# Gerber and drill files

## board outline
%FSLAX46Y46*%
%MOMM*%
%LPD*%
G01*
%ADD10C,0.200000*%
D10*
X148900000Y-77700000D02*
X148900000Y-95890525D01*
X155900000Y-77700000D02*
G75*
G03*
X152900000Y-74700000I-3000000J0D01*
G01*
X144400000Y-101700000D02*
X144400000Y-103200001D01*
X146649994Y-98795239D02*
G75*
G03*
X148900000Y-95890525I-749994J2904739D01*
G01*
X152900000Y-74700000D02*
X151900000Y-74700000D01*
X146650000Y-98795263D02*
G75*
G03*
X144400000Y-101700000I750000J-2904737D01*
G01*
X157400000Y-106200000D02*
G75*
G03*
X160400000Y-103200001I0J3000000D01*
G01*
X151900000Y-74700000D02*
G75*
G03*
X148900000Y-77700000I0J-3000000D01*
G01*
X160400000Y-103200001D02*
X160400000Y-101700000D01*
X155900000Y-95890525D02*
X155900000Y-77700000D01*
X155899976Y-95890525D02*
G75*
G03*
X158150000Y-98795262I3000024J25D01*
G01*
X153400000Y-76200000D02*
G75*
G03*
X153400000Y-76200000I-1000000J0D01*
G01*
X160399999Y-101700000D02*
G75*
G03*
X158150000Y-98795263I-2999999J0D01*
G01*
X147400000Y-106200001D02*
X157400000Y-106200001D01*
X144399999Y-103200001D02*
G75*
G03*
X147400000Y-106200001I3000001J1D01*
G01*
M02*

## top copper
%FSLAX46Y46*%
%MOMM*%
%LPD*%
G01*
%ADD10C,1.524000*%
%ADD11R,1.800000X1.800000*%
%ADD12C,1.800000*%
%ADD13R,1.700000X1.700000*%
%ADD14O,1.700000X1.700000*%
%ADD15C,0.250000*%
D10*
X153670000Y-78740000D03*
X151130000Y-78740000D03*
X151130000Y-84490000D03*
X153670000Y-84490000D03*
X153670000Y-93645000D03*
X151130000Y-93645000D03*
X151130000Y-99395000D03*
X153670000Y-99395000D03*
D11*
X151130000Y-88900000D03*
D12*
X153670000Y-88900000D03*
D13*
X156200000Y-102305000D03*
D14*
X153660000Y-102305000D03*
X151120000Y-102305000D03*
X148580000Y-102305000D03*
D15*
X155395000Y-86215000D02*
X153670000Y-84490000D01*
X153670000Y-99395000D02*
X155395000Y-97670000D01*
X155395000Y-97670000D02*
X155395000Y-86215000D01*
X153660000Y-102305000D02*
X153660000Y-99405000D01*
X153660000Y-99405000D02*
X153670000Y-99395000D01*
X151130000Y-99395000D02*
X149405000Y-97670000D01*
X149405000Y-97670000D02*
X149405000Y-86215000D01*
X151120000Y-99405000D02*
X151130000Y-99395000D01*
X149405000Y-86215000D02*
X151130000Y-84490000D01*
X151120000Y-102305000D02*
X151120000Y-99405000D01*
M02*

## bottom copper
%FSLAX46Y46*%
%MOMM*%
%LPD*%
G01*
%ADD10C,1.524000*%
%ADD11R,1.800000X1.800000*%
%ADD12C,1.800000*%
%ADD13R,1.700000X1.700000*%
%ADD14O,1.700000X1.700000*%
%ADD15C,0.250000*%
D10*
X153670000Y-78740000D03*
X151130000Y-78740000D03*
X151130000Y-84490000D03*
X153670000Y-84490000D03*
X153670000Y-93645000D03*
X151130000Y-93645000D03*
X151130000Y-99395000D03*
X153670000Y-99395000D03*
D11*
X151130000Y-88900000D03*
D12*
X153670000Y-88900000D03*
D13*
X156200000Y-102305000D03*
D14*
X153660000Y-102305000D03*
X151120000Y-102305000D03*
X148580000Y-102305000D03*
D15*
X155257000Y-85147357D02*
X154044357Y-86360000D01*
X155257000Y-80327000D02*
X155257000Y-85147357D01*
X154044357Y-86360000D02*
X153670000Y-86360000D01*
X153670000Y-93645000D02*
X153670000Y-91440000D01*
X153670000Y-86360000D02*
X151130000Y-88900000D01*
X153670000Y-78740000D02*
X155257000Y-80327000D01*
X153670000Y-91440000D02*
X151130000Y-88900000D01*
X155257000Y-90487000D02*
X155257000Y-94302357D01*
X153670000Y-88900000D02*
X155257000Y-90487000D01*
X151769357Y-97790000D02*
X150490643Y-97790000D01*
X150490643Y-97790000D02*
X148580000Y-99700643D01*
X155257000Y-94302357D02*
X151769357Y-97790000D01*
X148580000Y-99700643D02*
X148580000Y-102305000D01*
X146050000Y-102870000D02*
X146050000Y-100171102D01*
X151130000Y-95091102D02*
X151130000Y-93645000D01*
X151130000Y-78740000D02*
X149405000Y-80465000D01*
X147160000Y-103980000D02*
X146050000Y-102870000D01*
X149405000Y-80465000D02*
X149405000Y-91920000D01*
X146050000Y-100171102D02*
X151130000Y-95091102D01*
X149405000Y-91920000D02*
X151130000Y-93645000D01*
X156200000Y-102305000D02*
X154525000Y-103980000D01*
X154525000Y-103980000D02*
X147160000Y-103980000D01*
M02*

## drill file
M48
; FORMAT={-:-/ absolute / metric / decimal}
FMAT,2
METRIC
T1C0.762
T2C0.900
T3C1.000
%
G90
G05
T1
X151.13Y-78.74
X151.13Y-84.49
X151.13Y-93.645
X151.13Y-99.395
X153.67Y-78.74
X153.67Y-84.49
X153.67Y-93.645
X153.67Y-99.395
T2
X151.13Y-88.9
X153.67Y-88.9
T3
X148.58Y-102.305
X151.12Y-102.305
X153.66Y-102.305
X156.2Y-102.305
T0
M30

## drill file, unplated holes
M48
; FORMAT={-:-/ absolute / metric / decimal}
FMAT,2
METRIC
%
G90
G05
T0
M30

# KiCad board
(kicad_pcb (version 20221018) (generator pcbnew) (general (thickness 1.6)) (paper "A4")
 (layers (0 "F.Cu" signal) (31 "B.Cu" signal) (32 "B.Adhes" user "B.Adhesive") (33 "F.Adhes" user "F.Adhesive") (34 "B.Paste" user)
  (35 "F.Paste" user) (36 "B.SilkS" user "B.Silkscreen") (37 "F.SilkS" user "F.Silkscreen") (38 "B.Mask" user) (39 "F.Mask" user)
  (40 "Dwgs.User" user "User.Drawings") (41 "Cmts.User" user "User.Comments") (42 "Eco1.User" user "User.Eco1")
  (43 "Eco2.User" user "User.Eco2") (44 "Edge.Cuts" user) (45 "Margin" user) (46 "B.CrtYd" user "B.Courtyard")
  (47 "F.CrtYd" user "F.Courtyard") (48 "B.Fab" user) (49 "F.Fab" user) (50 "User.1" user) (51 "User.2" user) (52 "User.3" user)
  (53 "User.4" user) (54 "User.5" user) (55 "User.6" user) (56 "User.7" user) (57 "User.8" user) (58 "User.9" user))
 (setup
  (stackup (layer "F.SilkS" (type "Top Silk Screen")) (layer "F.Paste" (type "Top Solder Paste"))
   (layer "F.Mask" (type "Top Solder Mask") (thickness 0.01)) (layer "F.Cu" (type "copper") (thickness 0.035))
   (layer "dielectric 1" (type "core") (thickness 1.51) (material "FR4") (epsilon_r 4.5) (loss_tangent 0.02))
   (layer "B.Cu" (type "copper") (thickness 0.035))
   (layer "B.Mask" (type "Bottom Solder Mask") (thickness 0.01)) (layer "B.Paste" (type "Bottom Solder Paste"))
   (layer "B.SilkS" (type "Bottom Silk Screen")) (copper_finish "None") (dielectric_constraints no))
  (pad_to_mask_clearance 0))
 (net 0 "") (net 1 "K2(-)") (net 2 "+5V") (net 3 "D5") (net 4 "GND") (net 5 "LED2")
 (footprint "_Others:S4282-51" (layer "F.Cu") (at 152.4 81.615 -90)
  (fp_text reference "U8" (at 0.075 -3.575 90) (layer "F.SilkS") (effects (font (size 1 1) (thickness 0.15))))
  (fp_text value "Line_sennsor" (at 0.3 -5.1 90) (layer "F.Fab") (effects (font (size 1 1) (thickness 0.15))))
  (pad "1" thru_hole circle (at -2.875 -1.27 270) (size 1.524 1.524) (drill 0.762) (layers "*.Cu" "*.Mask") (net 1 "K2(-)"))
  (pad "2" thru_hole circle (at -2.875 1.27 270) (size 1.524 1.524) (drill 0.762) (layers "*.Cu" "*.Mask") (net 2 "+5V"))
  (pad "3" thru_hole circle (at 2.875 1.27 270) (size 1.524 1.524) (drill 0.762) (layers "*.Cu" "*.Mask") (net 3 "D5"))
  (pad "4" thru_hole circle (at 2.875 -1.27 270) (size 1.524 1.524) (drill 0.762) (layers "*.Cu" "*.Mask") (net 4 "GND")))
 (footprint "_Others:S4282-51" (layer "F.Cu") (at 152.4 96.52 -90)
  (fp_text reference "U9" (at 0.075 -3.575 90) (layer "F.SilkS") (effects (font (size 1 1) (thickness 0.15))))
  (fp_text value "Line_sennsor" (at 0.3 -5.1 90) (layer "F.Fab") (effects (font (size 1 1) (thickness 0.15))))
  (pad "1" thru_hole circle (at -2.875 -1.27 270) (size 1.524 1.524) (drill 0.762) (layers "*.Cu" "*.Mask") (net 1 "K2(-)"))
  (pad "2" thru_hole circle (at -2.875 1.27 270) (size 1.524 1.524) (drill 0.762) (layers "*.Cu" "*.Mask") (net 2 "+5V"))
  (pad "3" thru_hole circle (at 2.875 1.27 270) (size 1.524 1.524) (drill 0.762) (layers "*.Cu" "*.Mask") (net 3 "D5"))
  (pad "4" thru_hole circle (at 2.875 -1.27 270) (size 1.524 1.524) (drill 0.762) (layers "*.Cu" "*.Mask") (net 4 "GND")))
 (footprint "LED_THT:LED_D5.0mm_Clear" (layer "F.Cu") (at 151.13 88.9)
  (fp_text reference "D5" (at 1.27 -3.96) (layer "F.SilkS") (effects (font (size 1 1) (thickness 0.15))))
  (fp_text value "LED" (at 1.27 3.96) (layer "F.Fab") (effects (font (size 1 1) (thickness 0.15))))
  (pad "1" thru_hole rect (at 0 0) (size 1.8 1.8) (drill 0.9) (layers "*.Cu" "*.Mask") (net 1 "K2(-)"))
  (pad "2" thru_hole circle (at 2.54 0) (size 1.8 1.8) (drill 0.9) (layers "*.Cu" "*.Mask") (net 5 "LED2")))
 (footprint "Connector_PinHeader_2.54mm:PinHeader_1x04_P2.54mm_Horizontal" (layer "F.Cu") (at 156.2 102.305 -90)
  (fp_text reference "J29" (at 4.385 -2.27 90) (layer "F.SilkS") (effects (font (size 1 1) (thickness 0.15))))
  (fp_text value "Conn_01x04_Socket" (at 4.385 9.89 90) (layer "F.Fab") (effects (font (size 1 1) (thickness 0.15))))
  (pad "1" thru_hole rect (at 0 0 270) (size 1.7 1.7) (drill 1) (layers "*.Cu" "*.Mask") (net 2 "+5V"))
  (pad "2" thru_hole oval (at 0 2.54 270) (size 1.7 1.7) (drill 1) (layers "*.Cu" "*.Mask") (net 4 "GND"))
  (pad "3" thru_hole oval (at 0 5.08 270) (size 1.7 1.7) (drill 1) (layers "*.Cu" "*.Mask") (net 3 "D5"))
  (pad "4" thru_hole oval (at 0 7.62 270) (size 1.7 1.7) (drill 1) (layers "*.Cu" "*.Mask") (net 5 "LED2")))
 (gr_line (start 148.9 77.7) (end 148.9 95.890525) (stroke (width 0.2) (type solid)) (layer "Edge.Cuts"))
 (gr_arc (start 152.9 74.7) (mid 155.02132 75.57868) (end 155.9 77.7) (stroke (width 0.2) (type solid)) (layer "Edge.Cuts"))
 (gr_line (start 144.4 101.7) (end 144.4 103.200001) (stroke (width 0.2) (type solid)) (layer "Edge.Cuts"))
 (gr_arc (start 148.9 95.890525) (mid 148.271707 97.72764) (end 146.65 98.795263) (stroke (width 0.2) (type solid)) (layer "Edge.Cuts"))
 (gr_line (start 152.9 74.7) (end 151.9 74.7) (stroke (width 0.2) (type solid)) (layer "Edge.Cuts"))
 (gr_arc (start 144.4 101.7) (mid 145.028292 99.862883) (end 146.65 98.795263) (stroke (width 0.2) (type solid)) (layer "Edge.Cuts"))
 (gr_arc (start 160.4 103.200001) (mid 159.52132 105.321321) (end 157.4 106.200001) (stroke (width 0.2) (type solid)) (layer "Edge.Cuts"))
 (gr_arc (start 148.9 77.7) (mid 149.77868 75.57868) (end 151.9 74.7) (stroke (width 0.2) (type solid)) (layer "Edge.Cuts"))
 (gr_line (start 160.4 103.200001) (end 160.4 101.7) (stroke (width 0.2) (type solid)) (layer "Edge.Cuts"))
 (gr_line (start 155.9 95.890525) (end 155.9 77.7) (stroke (width 0.2) (type solid)) (layer "Edge.Cuts"))
 (gr_arc (start 158.15 98.795263) (mid 156.528291 97.727643) (end 155.9 95.890525) (stroke (width 0.2) (type solid)) (layer "Edge.Cuts"))
 (gr_circle (center 152.4 76.2) (end 151.4 76.2) (stroke (width 0.2) (type solid)) (fill none) (layer "Edge.Cuts"))
 (gr_arc (start 158.15 98.795263) (mid 159.771708 99.862883) (end 160.4 101.7) (stroke (width 0.2) (type solid)) (layer "Edge.Cuts"))
 (gr_line (start 147.4 106.200001) (end 157.4 106.200001) (stroke (width 0.2) (type solid)) (layer "Edge.Cuts"))
 (gr_arc (start 147.4 106.200001) (mid 145.27868 105.321321) (end 144.4 103.200001) (stroke (width 0.2) (type solid)) (layer "Edge.Cuts"))
 (segment (start 155.257 85.147357) (end 154.044357 86.36) (width 0.25) (layer "B.Cu") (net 1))
 (segment (start 155.257 80.327) (end 155.257 85.147357) (width 0.25) (layer "B.Cu") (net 1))
 (segment (start 154.044357 86.36) (end 153.67 86.36) (width 0.25) (layer "B.Cu") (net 1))
 (segment (start 153.67 93.645) (end 153.67 91.44) (width 0.25) (layer "B.Cu") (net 1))
 (segment (start 153.67 86.36) (end 151.13 88.9) (width 0.25) (layer "B.Cu") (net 1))
 (segment (start 153.67 78.74) (end 155.257 80.327) (width 0.25) (layer "B.Cu") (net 1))
 (segment (start 153.67 91.44) (end 151.13 88.9) (width 0.25) (layer "B.Cu") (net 1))
 (segment (start 155.257 90.487) (end 155.257 94.302357) (width 0.25) (layer "B.Cu") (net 5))
 (segment (start 153.67 88.9) (end 155.257 90.487) (width 0.25) (layer "B.Cu") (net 5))
 (segment (start 151.769357 97.79) (end 150.490643 97.79) (width 0.25) (layer "B.Cu") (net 5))
 (segment (start 150.490643 97.79) (end 148.58 99.700643) (width 0.25) (layer "B.Cu") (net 5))
 (segment (start 155.257 94.302357) (end 151.769357 97.79) (width 0.25) (layer "B.Cu") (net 5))
 (segment (start 148.58 99.700643) (end 148.58 102.305) (width 0.25) (layer "B.Cu") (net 5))
 (segment (start 146.05 102.87) (end 146.05 100.171102) (width 0.25) (layer "B.Cu") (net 2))
 (segment (start 151.13 95.091102) (end 151.13 93.645) (width 0.25) (layer "B.Cu") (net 2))
 (segment (start 151.13 78.74) (end 149.405 80.465) (width 0.25) (layer "B.Cu") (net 2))
 (segment (start 147.16 103.98) (end 146.05 102.87) (width 0.25) (layer "B.Cu") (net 2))
 (segment (start 149.405 80.465) (end 149.405 91.92) (width 0.25) (layer "B.Cu") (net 2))
 (segment (start 146.05 100.171102) (end 151.13 95.091102) (width 0.25) (layer "B.Cu") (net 2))
 (segment (start 149.405 91.92) (end 151.13 93.645) (width 0.25) (layer "B.Cu") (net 2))
 (segment (start 156.2 102.305) (end 154.525 103.98) (width 0.25) (layer "B.Cu") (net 2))
 (segment (start 154.525 103.98) (end 147.16 103.98) (width 0.25) (layer "B.Cu") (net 2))
 (segment (start 155.395 86.215) (end 153.67 84.49) (width 0.25) (layer "F.Cu") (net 4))
 (segment (start 153.67 99.395) (end 155.395 97.67) (width 0.25) (layer "F.Cu") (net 4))
 (segment (start 155.395 97.67) (end 155.395 86.215) (width 0.25) (layer "F.Cu") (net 4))
 (segment (start 153.66 102.305) (end 153.66 99.405) (width 0.25) (layer "F.Cu") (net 4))
 (segment (start 153.66 99.405) (end 153.67 99.395) (width 0.25) (layer "F.Cu") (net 4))
 (segment (start 151.13 99.395) (end 149.405 97.67) (width 0.25) (layer "F.Cu") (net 3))
 (segment (start 149.405 97.67) (end 149.405 86.215) (width 0.25) (layer "F.Cu") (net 3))
 (segment (start 151.12 99.405) (end 151.13 99.395) (width 0.25) (layer "F.Cu") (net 3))
 (segment (start 149.405 86.215) (end 151.13 84.49) (width 0.25) (layer "F.Cu") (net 3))
 (segment (start 151.12 102.305) (end 151.12 99.405) (width 0.25) (layer "F.Cu") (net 3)))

